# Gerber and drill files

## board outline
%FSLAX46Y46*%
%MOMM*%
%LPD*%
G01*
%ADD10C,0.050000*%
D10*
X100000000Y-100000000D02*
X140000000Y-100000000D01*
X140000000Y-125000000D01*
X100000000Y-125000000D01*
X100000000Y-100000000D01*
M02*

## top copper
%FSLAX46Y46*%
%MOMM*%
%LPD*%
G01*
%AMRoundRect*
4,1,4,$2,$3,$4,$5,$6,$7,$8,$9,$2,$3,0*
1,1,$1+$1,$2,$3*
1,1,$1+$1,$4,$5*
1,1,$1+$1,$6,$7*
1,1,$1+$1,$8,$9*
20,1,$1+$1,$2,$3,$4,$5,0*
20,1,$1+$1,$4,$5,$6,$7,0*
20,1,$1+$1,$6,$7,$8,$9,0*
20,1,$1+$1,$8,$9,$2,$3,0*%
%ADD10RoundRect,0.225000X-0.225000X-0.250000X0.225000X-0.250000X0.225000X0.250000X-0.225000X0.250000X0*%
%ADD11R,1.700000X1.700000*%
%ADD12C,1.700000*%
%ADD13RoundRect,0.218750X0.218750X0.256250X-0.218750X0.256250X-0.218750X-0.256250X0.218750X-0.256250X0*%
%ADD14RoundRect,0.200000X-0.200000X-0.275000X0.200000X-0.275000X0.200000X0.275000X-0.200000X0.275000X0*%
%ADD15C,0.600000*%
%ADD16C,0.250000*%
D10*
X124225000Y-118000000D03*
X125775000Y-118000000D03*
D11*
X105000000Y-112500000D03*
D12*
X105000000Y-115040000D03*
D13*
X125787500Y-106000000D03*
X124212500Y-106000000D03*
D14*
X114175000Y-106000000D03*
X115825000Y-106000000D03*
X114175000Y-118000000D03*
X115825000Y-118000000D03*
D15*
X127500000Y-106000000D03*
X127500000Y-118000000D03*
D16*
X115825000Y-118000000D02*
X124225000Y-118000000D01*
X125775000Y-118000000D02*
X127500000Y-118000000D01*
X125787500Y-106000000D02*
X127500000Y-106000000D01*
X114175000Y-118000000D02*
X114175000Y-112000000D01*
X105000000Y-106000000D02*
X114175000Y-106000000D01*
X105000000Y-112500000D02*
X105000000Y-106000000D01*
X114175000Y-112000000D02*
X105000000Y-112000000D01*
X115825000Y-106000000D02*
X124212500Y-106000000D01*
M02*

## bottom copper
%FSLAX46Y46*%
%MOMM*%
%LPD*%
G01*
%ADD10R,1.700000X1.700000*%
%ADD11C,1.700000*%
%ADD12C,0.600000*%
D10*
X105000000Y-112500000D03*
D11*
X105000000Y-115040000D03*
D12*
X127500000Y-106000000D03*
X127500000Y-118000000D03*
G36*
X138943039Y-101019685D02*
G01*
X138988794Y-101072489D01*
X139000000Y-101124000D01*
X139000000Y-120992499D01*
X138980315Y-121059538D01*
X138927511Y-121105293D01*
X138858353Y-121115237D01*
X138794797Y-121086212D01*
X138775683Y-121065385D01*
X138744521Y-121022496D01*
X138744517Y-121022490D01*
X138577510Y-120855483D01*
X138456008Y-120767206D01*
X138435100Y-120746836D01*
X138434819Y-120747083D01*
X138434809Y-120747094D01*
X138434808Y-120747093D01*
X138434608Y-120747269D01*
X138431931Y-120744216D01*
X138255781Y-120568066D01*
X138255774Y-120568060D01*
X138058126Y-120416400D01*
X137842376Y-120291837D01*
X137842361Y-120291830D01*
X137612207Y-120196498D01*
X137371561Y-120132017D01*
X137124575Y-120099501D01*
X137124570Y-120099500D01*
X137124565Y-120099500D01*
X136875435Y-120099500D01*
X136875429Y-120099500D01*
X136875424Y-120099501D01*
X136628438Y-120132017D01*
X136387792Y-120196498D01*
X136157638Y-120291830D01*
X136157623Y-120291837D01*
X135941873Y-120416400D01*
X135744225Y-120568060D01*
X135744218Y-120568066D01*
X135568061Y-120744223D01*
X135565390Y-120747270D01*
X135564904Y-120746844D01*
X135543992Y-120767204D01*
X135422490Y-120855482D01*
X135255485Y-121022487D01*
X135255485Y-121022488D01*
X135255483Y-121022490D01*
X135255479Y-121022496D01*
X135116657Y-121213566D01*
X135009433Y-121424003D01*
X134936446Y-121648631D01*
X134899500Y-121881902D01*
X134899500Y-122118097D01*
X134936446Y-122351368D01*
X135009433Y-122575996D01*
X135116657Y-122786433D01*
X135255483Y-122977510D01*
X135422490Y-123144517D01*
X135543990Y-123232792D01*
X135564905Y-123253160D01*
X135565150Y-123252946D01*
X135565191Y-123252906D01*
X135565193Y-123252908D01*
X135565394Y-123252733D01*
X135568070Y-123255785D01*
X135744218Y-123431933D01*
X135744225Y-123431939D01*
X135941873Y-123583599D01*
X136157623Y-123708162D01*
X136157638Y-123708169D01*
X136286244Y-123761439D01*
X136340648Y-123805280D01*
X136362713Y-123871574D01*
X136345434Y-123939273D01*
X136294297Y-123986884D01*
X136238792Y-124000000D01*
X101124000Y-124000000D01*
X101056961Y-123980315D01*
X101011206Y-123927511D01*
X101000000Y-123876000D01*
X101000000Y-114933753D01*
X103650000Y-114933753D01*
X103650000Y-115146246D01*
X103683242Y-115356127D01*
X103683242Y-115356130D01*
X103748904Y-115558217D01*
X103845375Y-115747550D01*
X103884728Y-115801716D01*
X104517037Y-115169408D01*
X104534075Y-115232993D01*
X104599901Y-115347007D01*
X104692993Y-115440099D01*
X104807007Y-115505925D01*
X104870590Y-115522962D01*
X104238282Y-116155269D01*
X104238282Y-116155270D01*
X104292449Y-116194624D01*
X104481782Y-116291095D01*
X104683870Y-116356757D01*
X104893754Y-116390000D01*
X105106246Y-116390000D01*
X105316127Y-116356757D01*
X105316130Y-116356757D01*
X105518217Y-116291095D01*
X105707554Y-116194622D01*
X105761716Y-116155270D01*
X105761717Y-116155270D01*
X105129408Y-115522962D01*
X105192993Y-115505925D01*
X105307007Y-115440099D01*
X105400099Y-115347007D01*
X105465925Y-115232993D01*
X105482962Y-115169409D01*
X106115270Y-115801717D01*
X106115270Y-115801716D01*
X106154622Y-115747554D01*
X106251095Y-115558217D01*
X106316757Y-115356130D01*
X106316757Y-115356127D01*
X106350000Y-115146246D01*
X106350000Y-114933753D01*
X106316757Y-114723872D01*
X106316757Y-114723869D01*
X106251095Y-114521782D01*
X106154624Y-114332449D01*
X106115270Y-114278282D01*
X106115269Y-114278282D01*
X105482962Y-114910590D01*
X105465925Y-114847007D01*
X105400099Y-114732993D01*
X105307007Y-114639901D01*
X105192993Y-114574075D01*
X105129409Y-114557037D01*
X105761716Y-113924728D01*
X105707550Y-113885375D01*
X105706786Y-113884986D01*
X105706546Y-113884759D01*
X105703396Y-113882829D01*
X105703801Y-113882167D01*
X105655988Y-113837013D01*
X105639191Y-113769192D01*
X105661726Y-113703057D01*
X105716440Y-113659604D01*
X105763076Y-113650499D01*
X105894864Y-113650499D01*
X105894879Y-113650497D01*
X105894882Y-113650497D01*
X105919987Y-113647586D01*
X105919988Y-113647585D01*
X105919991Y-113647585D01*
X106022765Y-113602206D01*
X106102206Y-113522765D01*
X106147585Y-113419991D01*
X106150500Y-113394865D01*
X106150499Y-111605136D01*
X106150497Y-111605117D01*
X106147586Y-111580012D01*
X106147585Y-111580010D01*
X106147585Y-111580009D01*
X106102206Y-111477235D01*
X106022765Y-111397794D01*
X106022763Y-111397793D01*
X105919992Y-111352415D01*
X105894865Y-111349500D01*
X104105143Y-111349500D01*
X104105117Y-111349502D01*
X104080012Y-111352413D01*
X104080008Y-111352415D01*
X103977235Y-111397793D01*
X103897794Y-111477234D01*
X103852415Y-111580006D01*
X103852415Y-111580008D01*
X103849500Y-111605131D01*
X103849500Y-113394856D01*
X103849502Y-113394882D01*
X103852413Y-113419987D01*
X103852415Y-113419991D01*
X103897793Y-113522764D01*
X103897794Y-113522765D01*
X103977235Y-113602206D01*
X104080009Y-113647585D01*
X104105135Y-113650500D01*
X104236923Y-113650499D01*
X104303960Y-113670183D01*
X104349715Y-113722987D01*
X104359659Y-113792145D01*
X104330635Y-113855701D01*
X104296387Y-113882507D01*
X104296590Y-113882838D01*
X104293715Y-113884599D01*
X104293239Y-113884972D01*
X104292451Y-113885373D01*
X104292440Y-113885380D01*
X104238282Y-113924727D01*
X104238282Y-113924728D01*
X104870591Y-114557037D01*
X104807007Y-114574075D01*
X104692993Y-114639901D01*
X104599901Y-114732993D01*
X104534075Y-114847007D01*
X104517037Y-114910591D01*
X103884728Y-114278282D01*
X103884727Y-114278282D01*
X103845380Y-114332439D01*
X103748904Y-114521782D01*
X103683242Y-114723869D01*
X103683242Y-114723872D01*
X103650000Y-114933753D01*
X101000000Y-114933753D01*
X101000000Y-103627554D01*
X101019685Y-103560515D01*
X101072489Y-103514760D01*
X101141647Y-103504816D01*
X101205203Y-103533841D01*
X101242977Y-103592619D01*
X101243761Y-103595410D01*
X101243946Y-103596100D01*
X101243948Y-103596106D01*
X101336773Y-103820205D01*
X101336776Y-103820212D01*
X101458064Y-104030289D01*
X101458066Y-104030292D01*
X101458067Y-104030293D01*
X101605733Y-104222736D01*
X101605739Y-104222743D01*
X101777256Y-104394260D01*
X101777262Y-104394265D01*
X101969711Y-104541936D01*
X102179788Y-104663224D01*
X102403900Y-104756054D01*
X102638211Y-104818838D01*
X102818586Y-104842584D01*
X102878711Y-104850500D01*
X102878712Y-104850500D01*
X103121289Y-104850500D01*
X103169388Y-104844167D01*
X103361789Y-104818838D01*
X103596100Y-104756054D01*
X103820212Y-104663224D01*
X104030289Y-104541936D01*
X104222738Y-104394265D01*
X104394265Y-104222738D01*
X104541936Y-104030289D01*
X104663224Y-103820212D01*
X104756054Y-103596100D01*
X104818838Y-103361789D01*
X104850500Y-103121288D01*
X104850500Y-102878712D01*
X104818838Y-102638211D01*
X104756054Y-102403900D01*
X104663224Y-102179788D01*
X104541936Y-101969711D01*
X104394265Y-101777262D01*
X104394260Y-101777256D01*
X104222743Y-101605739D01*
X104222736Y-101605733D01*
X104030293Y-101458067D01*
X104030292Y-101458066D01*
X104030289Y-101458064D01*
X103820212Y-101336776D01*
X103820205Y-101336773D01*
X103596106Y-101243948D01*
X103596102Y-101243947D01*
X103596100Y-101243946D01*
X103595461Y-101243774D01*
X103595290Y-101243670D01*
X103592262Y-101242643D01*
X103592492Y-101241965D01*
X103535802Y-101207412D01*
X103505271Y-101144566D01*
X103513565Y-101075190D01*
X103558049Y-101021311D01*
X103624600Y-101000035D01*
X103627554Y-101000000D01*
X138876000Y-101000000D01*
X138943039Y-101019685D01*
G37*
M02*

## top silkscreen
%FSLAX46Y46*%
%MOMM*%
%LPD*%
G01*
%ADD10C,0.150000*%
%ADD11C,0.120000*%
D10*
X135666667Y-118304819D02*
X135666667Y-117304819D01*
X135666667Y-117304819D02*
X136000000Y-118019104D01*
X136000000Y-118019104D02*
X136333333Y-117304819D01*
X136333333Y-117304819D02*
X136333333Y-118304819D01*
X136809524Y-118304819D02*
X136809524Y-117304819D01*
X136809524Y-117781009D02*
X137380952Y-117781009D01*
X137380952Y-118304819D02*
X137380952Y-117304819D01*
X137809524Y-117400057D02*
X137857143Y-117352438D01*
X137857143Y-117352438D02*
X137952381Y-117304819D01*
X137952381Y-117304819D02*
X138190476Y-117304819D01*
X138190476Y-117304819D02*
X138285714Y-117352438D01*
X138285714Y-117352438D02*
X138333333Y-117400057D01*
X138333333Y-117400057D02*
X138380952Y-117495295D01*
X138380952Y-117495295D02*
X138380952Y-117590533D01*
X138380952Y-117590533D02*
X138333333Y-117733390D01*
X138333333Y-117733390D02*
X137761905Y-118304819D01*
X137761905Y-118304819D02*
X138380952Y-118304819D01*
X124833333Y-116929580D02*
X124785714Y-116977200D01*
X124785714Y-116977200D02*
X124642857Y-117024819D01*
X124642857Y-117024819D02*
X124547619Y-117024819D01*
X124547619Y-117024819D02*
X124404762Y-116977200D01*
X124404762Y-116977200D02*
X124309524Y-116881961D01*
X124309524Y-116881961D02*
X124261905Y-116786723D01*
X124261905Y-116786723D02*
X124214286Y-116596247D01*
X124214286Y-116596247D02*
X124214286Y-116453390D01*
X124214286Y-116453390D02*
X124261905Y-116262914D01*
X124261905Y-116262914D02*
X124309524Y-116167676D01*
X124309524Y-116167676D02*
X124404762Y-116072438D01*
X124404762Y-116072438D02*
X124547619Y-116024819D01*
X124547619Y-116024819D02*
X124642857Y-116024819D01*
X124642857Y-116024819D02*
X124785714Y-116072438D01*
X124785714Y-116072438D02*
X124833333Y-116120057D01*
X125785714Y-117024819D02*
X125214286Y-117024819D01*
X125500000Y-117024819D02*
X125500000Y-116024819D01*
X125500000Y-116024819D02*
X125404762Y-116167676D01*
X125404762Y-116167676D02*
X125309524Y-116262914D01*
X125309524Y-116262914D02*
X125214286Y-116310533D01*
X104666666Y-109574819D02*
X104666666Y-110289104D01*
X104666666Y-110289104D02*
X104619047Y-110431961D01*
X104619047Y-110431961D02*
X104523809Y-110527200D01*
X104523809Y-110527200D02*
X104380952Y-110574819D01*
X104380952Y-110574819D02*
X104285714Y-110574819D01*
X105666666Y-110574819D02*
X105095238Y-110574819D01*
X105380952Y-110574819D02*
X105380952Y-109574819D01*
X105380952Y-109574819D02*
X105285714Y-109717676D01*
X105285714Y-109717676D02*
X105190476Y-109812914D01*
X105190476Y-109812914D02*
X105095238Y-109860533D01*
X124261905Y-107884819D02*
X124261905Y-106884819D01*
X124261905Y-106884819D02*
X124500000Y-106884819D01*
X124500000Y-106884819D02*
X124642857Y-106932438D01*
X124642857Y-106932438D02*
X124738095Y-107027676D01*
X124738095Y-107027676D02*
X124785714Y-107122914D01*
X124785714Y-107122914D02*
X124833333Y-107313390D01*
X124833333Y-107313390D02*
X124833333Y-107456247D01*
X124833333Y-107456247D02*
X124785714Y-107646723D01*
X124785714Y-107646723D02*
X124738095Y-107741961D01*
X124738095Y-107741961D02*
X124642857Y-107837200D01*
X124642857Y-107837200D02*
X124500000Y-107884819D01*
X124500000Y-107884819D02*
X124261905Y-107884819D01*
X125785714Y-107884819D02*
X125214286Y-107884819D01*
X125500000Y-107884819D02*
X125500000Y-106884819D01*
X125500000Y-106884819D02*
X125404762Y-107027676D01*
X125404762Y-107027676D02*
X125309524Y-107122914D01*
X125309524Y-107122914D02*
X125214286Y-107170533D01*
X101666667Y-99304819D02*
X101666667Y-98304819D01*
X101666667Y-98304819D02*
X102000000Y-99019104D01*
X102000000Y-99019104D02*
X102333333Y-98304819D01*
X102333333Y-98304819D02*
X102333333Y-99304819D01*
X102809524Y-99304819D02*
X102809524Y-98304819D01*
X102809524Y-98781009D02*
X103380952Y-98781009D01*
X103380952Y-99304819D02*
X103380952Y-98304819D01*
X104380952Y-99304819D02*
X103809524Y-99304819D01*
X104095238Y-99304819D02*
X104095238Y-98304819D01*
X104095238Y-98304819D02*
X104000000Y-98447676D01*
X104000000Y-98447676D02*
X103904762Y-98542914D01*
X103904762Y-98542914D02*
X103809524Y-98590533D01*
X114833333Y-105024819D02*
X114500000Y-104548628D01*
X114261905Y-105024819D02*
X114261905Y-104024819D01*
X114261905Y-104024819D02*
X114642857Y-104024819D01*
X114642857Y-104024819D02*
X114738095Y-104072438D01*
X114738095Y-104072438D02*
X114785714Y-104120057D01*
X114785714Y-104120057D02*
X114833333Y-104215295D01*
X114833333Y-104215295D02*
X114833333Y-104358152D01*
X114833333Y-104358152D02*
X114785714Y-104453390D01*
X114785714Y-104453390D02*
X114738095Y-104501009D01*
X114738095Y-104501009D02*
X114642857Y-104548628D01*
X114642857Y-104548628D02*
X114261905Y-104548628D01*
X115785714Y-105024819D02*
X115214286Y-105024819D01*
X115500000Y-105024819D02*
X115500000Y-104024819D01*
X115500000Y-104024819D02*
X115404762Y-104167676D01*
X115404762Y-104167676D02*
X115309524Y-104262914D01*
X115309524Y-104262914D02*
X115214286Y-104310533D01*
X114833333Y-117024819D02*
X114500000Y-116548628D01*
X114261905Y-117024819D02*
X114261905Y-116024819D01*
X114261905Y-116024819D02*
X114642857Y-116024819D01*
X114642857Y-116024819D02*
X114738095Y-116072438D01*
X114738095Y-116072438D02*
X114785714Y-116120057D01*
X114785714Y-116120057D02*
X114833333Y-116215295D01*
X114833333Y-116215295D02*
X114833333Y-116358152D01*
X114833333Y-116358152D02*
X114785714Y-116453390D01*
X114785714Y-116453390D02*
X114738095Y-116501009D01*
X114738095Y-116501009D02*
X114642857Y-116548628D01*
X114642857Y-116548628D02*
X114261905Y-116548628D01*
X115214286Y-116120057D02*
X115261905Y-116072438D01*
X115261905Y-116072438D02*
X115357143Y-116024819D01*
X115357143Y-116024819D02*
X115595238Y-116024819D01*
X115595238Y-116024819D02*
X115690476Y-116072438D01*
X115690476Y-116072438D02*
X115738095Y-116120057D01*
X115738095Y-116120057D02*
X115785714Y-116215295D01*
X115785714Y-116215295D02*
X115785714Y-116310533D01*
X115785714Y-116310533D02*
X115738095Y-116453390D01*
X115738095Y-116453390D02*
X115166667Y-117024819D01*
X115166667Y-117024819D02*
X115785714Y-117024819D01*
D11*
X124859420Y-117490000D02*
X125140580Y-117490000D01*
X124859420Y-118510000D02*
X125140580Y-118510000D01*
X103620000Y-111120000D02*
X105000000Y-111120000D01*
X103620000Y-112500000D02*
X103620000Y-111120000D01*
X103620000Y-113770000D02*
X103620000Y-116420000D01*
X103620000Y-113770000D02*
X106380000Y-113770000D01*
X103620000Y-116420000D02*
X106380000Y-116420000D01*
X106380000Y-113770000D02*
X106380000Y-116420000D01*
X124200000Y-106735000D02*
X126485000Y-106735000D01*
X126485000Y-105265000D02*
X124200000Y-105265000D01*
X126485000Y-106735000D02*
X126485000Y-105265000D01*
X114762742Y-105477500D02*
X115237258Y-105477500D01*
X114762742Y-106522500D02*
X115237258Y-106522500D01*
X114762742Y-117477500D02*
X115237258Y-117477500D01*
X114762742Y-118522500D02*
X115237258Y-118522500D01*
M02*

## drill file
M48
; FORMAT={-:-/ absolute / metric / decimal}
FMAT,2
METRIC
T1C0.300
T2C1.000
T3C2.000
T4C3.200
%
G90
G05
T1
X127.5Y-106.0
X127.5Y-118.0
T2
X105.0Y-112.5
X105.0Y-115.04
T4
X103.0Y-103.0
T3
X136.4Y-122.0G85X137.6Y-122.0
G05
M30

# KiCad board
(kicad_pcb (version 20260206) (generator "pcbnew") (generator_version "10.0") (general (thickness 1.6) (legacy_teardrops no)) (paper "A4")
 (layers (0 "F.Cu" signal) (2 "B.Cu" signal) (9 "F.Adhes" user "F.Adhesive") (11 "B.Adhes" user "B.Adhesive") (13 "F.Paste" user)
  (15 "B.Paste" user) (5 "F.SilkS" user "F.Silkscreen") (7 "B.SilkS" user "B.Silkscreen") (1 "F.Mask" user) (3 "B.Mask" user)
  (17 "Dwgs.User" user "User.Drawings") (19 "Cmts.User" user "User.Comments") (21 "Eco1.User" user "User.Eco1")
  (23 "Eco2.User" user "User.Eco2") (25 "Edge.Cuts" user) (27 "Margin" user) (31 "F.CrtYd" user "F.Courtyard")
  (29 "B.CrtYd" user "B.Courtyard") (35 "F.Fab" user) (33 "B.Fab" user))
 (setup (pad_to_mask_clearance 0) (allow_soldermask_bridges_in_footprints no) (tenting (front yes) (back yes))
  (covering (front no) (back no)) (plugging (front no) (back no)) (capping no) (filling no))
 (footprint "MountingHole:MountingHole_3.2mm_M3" (layer "F.Cu") (at 137 122)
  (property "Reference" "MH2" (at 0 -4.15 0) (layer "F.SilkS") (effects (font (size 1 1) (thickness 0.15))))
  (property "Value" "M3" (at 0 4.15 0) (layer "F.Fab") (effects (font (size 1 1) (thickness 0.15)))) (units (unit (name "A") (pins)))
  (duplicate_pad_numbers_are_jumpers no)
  (pad "" np_thru_hole circle (at 0 0) (size 3.2 3.2) (drill oval 3.2 2.0) (layers "*.Cu" "*.Mask")))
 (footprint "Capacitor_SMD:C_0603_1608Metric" (layer "F.Cu") (at 125 118)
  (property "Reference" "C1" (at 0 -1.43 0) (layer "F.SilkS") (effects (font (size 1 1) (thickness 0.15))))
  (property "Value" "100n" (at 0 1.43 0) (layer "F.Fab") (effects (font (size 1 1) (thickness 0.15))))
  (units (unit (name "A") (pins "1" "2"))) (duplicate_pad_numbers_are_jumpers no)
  (fp_line (start -0.14058 -0.51) (end 0.14058 -0.51) (stroke (width 0.12) (type solid)) (layer "F.SilkS"))
  (fp_line (start -0.14058 0.51) (end 0.14058 0.51) (stroke (width 0.12) (type solid)) (layer "F.SilkS"))
  (pad "1" smd roundrect (at -0.775 0) (size 0.9 0.95) (layers "F.Cu" "F.Mask" "F.Paste") (roundrect_rratio 0.25) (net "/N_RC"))
  (pad "2" smd roundrect (at 0.775 0) (size 0.9 0.95) (layers "F.Cu" "F.Mask" "F.Paste") (roundrect_rratio 0.25) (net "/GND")))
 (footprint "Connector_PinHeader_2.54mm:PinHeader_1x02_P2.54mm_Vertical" (layer "F.Cu") (at 105 112.5)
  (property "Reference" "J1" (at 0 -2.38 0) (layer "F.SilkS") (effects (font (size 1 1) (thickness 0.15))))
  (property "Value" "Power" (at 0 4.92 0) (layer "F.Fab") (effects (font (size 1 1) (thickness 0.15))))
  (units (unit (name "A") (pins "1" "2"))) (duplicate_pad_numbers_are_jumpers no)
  (fp_line (start -1.38 -1.38) (end 0 -1.38) (stroke (width 0.12) (type solid)) (layer "F.SilkS"))
  (fp_line (start -1.38 0) (end -1.38 -1.38) (stroke (width 0.12) (type solid)) (layer "F.SilkS"))
  (fp_line (start -1.38 1.27) (end -1.38 3.92) (stroke (width 0.12) (type solid)) (layer "F.SilkS"))
  (fp_line (start -1.38 1.27) (end 1.38 1.27) (stroke (width 0.12) (type solid)) (layer "F.SilkS"))
  (fp_line (start -1.38 3.92) (end 1.38 3.92) (stroke (width 0.12) (type solid)) (layer "F.SilkS"))
  (fp_line (start 1.38 1.27) (end 1.38 3.92) (stroke (width 0.12) (type solid)) (layer "F.SilkS"))
  (pad "1" thru_hole rect (at 0 0) (size 1.7 1.7) (drill 1) (layers "*.Cu" "*.Mask") (remove_unused_layers no) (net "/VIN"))
  (pad "2" thru_hole circle (at 0 2.54) (size 1.7 1.7) (drill 1) (layers "*.Cu" "*.Mask") (remove_unused_layers no) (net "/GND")))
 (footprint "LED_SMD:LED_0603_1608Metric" (layer "F.Cu") (at 125 106 180)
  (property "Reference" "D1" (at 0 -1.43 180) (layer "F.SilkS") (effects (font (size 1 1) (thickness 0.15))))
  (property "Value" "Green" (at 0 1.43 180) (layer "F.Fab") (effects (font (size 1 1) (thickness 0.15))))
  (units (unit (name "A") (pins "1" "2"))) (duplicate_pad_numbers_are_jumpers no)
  (fp_line (start 0.8 -0.735) (end -1.485 -0.735) (stroke (width 0.12) (type solid)) (layer "F.SilkS"))
  (fp_line (start -1.485 0.735) (end 0.8 0.735) (stroke (width 0.12) (type solid)) (layer "F.SilkS"))
  (fp_line (start -1.485 -0.735) (end -1.485 0.735) (stroke (width 0.12) (type solid)) (layer "F.SilkS"))
  (pad "1" smd roundrect (at -0.7875 0 180) (size 0.875 0.95) (layers "F.Cu" "F.Mask" "F.Paste") (roundrect_rratio 0.25) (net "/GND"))
  (pad "2" smd roundrect (at 0.7875 0 180) (size 0.875 0.95) (layers "F.Cu" "F.Mask" "F.Paste") (roundrect_rratio 0.25) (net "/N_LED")))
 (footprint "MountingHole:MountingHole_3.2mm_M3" (layer "F.Cu") (at 103 103)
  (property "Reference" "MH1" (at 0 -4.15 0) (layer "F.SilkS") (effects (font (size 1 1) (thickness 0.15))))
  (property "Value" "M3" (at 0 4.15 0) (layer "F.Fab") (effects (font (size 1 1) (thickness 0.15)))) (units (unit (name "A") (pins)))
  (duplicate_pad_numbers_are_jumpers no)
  (pad "" np_thru_hole circle (at 0 0) (size 3.2 3.2) (drill 3.2) (layers "*.Cu" "*.Mask")))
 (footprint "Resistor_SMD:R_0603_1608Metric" (layer "F.Cu") (at 115 106)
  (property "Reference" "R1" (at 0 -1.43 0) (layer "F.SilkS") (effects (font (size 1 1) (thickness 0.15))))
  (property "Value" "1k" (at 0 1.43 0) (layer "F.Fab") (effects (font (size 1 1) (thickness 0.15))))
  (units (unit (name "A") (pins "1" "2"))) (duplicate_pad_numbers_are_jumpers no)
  (fp_line (start -0.237258 -0.5225) (end 0.237258 -0.5225) (stroke (width 0.12) (type solid)) (layer "F.SilkS"))
  (fp_line (start -0.237258 0.5225) (end 0.237258 0.5225) (stroke (width 0.12) (type solid)) (layer "F.SilkS"))
  (pad "1" smd roundrect (at -0.825 0) (size 0.8 0.95) (layers "F.Cu" "F.Mask" "F.Paste") (roundrect_rratio 0.25) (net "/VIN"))
  (pad "2" smd roundrect (at 0.825 0) (size 0.8 0.95) (layers "F.Cu" "F.Mask" "F.Paste") (roundrect_rratio 0.25) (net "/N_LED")))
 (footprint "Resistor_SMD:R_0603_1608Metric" (layer "F.Cu") (at 115 118)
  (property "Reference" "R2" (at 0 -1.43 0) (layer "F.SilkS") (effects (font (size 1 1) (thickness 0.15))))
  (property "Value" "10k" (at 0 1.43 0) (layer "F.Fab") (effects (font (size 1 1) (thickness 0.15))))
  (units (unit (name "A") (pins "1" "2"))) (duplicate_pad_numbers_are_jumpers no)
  (fp_line (start -0.237258 -0.5225) (end 0.237258 -0.5225) (stroke (width 0.12) (type solid)) (layer "F.SilkS"))
  (fp_line (start -0.237258 0.5225) (end 0.237258 0.5225) (stroke (width 0.12) (type solid)) (layer "F.SilkS"))
  (pad "1" smd roundrect (at -0.825 0) (size 0.8 0.95) (layers "F.Cu" "F.Mask" "F.Paste") (roundrect_rratio 0.25) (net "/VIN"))
  (pad "2" smd roundrect (at 0.825 0) (size 0.8 0.95) (layers "F.Cu" "F.Mask" "F.Paste") (roundrect_rratio 0.25) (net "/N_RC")))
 (gr_rect (start 100 100) (end 140 125) (stroke (width 0.05) (type default)) (fill no) (layer "Edge.Cuts"))
 (segment (start 115.825 118) (end 124.225 118) (width 0.25) (layer "F.Cu") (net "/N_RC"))
 (segment (start 125.775 118) (end 127.5 118) (width 0.25) (layer "F.Cu") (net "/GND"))
 (segment (start 125.7875 106) (end 127.5 106) (width 0.25) (layer "F.Cu") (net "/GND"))
 (via (at 127.5 106) (size 0.6) (drill 0.3) (layers "F.Cu" "B.Cu") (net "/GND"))
 (via (at 127.5 118) (size 0.6) (drill 0.3) (layers "F.Cu" "B.Cu") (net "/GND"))
 (segment (start 114.175 118) (end 114.175 112) (width 0.25) (layer "F.Cu") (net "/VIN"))
 (segment (start 105 106) (end 114.175 106) (width 0.25) (layer "F.Cu") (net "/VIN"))
 (segment (start 105 112.5) (end 105 106) (width 0.25) (layer "F.Cu") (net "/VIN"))
 (segment (start 114.175 112) (end 105 112) (width 0.25) (layer "F.Cu") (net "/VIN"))
 (segment (start 115.825 106) (end 124.2125 106) (width 0.25) (layer "F.Cu") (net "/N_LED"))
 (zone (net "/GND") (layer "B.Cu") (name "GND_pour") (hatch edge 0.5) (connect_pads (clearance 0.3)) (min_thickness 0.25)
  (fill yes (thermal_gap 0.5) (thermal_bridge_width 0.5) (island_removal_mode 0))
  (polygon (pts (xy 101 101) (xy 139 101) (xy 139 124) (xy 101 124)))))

